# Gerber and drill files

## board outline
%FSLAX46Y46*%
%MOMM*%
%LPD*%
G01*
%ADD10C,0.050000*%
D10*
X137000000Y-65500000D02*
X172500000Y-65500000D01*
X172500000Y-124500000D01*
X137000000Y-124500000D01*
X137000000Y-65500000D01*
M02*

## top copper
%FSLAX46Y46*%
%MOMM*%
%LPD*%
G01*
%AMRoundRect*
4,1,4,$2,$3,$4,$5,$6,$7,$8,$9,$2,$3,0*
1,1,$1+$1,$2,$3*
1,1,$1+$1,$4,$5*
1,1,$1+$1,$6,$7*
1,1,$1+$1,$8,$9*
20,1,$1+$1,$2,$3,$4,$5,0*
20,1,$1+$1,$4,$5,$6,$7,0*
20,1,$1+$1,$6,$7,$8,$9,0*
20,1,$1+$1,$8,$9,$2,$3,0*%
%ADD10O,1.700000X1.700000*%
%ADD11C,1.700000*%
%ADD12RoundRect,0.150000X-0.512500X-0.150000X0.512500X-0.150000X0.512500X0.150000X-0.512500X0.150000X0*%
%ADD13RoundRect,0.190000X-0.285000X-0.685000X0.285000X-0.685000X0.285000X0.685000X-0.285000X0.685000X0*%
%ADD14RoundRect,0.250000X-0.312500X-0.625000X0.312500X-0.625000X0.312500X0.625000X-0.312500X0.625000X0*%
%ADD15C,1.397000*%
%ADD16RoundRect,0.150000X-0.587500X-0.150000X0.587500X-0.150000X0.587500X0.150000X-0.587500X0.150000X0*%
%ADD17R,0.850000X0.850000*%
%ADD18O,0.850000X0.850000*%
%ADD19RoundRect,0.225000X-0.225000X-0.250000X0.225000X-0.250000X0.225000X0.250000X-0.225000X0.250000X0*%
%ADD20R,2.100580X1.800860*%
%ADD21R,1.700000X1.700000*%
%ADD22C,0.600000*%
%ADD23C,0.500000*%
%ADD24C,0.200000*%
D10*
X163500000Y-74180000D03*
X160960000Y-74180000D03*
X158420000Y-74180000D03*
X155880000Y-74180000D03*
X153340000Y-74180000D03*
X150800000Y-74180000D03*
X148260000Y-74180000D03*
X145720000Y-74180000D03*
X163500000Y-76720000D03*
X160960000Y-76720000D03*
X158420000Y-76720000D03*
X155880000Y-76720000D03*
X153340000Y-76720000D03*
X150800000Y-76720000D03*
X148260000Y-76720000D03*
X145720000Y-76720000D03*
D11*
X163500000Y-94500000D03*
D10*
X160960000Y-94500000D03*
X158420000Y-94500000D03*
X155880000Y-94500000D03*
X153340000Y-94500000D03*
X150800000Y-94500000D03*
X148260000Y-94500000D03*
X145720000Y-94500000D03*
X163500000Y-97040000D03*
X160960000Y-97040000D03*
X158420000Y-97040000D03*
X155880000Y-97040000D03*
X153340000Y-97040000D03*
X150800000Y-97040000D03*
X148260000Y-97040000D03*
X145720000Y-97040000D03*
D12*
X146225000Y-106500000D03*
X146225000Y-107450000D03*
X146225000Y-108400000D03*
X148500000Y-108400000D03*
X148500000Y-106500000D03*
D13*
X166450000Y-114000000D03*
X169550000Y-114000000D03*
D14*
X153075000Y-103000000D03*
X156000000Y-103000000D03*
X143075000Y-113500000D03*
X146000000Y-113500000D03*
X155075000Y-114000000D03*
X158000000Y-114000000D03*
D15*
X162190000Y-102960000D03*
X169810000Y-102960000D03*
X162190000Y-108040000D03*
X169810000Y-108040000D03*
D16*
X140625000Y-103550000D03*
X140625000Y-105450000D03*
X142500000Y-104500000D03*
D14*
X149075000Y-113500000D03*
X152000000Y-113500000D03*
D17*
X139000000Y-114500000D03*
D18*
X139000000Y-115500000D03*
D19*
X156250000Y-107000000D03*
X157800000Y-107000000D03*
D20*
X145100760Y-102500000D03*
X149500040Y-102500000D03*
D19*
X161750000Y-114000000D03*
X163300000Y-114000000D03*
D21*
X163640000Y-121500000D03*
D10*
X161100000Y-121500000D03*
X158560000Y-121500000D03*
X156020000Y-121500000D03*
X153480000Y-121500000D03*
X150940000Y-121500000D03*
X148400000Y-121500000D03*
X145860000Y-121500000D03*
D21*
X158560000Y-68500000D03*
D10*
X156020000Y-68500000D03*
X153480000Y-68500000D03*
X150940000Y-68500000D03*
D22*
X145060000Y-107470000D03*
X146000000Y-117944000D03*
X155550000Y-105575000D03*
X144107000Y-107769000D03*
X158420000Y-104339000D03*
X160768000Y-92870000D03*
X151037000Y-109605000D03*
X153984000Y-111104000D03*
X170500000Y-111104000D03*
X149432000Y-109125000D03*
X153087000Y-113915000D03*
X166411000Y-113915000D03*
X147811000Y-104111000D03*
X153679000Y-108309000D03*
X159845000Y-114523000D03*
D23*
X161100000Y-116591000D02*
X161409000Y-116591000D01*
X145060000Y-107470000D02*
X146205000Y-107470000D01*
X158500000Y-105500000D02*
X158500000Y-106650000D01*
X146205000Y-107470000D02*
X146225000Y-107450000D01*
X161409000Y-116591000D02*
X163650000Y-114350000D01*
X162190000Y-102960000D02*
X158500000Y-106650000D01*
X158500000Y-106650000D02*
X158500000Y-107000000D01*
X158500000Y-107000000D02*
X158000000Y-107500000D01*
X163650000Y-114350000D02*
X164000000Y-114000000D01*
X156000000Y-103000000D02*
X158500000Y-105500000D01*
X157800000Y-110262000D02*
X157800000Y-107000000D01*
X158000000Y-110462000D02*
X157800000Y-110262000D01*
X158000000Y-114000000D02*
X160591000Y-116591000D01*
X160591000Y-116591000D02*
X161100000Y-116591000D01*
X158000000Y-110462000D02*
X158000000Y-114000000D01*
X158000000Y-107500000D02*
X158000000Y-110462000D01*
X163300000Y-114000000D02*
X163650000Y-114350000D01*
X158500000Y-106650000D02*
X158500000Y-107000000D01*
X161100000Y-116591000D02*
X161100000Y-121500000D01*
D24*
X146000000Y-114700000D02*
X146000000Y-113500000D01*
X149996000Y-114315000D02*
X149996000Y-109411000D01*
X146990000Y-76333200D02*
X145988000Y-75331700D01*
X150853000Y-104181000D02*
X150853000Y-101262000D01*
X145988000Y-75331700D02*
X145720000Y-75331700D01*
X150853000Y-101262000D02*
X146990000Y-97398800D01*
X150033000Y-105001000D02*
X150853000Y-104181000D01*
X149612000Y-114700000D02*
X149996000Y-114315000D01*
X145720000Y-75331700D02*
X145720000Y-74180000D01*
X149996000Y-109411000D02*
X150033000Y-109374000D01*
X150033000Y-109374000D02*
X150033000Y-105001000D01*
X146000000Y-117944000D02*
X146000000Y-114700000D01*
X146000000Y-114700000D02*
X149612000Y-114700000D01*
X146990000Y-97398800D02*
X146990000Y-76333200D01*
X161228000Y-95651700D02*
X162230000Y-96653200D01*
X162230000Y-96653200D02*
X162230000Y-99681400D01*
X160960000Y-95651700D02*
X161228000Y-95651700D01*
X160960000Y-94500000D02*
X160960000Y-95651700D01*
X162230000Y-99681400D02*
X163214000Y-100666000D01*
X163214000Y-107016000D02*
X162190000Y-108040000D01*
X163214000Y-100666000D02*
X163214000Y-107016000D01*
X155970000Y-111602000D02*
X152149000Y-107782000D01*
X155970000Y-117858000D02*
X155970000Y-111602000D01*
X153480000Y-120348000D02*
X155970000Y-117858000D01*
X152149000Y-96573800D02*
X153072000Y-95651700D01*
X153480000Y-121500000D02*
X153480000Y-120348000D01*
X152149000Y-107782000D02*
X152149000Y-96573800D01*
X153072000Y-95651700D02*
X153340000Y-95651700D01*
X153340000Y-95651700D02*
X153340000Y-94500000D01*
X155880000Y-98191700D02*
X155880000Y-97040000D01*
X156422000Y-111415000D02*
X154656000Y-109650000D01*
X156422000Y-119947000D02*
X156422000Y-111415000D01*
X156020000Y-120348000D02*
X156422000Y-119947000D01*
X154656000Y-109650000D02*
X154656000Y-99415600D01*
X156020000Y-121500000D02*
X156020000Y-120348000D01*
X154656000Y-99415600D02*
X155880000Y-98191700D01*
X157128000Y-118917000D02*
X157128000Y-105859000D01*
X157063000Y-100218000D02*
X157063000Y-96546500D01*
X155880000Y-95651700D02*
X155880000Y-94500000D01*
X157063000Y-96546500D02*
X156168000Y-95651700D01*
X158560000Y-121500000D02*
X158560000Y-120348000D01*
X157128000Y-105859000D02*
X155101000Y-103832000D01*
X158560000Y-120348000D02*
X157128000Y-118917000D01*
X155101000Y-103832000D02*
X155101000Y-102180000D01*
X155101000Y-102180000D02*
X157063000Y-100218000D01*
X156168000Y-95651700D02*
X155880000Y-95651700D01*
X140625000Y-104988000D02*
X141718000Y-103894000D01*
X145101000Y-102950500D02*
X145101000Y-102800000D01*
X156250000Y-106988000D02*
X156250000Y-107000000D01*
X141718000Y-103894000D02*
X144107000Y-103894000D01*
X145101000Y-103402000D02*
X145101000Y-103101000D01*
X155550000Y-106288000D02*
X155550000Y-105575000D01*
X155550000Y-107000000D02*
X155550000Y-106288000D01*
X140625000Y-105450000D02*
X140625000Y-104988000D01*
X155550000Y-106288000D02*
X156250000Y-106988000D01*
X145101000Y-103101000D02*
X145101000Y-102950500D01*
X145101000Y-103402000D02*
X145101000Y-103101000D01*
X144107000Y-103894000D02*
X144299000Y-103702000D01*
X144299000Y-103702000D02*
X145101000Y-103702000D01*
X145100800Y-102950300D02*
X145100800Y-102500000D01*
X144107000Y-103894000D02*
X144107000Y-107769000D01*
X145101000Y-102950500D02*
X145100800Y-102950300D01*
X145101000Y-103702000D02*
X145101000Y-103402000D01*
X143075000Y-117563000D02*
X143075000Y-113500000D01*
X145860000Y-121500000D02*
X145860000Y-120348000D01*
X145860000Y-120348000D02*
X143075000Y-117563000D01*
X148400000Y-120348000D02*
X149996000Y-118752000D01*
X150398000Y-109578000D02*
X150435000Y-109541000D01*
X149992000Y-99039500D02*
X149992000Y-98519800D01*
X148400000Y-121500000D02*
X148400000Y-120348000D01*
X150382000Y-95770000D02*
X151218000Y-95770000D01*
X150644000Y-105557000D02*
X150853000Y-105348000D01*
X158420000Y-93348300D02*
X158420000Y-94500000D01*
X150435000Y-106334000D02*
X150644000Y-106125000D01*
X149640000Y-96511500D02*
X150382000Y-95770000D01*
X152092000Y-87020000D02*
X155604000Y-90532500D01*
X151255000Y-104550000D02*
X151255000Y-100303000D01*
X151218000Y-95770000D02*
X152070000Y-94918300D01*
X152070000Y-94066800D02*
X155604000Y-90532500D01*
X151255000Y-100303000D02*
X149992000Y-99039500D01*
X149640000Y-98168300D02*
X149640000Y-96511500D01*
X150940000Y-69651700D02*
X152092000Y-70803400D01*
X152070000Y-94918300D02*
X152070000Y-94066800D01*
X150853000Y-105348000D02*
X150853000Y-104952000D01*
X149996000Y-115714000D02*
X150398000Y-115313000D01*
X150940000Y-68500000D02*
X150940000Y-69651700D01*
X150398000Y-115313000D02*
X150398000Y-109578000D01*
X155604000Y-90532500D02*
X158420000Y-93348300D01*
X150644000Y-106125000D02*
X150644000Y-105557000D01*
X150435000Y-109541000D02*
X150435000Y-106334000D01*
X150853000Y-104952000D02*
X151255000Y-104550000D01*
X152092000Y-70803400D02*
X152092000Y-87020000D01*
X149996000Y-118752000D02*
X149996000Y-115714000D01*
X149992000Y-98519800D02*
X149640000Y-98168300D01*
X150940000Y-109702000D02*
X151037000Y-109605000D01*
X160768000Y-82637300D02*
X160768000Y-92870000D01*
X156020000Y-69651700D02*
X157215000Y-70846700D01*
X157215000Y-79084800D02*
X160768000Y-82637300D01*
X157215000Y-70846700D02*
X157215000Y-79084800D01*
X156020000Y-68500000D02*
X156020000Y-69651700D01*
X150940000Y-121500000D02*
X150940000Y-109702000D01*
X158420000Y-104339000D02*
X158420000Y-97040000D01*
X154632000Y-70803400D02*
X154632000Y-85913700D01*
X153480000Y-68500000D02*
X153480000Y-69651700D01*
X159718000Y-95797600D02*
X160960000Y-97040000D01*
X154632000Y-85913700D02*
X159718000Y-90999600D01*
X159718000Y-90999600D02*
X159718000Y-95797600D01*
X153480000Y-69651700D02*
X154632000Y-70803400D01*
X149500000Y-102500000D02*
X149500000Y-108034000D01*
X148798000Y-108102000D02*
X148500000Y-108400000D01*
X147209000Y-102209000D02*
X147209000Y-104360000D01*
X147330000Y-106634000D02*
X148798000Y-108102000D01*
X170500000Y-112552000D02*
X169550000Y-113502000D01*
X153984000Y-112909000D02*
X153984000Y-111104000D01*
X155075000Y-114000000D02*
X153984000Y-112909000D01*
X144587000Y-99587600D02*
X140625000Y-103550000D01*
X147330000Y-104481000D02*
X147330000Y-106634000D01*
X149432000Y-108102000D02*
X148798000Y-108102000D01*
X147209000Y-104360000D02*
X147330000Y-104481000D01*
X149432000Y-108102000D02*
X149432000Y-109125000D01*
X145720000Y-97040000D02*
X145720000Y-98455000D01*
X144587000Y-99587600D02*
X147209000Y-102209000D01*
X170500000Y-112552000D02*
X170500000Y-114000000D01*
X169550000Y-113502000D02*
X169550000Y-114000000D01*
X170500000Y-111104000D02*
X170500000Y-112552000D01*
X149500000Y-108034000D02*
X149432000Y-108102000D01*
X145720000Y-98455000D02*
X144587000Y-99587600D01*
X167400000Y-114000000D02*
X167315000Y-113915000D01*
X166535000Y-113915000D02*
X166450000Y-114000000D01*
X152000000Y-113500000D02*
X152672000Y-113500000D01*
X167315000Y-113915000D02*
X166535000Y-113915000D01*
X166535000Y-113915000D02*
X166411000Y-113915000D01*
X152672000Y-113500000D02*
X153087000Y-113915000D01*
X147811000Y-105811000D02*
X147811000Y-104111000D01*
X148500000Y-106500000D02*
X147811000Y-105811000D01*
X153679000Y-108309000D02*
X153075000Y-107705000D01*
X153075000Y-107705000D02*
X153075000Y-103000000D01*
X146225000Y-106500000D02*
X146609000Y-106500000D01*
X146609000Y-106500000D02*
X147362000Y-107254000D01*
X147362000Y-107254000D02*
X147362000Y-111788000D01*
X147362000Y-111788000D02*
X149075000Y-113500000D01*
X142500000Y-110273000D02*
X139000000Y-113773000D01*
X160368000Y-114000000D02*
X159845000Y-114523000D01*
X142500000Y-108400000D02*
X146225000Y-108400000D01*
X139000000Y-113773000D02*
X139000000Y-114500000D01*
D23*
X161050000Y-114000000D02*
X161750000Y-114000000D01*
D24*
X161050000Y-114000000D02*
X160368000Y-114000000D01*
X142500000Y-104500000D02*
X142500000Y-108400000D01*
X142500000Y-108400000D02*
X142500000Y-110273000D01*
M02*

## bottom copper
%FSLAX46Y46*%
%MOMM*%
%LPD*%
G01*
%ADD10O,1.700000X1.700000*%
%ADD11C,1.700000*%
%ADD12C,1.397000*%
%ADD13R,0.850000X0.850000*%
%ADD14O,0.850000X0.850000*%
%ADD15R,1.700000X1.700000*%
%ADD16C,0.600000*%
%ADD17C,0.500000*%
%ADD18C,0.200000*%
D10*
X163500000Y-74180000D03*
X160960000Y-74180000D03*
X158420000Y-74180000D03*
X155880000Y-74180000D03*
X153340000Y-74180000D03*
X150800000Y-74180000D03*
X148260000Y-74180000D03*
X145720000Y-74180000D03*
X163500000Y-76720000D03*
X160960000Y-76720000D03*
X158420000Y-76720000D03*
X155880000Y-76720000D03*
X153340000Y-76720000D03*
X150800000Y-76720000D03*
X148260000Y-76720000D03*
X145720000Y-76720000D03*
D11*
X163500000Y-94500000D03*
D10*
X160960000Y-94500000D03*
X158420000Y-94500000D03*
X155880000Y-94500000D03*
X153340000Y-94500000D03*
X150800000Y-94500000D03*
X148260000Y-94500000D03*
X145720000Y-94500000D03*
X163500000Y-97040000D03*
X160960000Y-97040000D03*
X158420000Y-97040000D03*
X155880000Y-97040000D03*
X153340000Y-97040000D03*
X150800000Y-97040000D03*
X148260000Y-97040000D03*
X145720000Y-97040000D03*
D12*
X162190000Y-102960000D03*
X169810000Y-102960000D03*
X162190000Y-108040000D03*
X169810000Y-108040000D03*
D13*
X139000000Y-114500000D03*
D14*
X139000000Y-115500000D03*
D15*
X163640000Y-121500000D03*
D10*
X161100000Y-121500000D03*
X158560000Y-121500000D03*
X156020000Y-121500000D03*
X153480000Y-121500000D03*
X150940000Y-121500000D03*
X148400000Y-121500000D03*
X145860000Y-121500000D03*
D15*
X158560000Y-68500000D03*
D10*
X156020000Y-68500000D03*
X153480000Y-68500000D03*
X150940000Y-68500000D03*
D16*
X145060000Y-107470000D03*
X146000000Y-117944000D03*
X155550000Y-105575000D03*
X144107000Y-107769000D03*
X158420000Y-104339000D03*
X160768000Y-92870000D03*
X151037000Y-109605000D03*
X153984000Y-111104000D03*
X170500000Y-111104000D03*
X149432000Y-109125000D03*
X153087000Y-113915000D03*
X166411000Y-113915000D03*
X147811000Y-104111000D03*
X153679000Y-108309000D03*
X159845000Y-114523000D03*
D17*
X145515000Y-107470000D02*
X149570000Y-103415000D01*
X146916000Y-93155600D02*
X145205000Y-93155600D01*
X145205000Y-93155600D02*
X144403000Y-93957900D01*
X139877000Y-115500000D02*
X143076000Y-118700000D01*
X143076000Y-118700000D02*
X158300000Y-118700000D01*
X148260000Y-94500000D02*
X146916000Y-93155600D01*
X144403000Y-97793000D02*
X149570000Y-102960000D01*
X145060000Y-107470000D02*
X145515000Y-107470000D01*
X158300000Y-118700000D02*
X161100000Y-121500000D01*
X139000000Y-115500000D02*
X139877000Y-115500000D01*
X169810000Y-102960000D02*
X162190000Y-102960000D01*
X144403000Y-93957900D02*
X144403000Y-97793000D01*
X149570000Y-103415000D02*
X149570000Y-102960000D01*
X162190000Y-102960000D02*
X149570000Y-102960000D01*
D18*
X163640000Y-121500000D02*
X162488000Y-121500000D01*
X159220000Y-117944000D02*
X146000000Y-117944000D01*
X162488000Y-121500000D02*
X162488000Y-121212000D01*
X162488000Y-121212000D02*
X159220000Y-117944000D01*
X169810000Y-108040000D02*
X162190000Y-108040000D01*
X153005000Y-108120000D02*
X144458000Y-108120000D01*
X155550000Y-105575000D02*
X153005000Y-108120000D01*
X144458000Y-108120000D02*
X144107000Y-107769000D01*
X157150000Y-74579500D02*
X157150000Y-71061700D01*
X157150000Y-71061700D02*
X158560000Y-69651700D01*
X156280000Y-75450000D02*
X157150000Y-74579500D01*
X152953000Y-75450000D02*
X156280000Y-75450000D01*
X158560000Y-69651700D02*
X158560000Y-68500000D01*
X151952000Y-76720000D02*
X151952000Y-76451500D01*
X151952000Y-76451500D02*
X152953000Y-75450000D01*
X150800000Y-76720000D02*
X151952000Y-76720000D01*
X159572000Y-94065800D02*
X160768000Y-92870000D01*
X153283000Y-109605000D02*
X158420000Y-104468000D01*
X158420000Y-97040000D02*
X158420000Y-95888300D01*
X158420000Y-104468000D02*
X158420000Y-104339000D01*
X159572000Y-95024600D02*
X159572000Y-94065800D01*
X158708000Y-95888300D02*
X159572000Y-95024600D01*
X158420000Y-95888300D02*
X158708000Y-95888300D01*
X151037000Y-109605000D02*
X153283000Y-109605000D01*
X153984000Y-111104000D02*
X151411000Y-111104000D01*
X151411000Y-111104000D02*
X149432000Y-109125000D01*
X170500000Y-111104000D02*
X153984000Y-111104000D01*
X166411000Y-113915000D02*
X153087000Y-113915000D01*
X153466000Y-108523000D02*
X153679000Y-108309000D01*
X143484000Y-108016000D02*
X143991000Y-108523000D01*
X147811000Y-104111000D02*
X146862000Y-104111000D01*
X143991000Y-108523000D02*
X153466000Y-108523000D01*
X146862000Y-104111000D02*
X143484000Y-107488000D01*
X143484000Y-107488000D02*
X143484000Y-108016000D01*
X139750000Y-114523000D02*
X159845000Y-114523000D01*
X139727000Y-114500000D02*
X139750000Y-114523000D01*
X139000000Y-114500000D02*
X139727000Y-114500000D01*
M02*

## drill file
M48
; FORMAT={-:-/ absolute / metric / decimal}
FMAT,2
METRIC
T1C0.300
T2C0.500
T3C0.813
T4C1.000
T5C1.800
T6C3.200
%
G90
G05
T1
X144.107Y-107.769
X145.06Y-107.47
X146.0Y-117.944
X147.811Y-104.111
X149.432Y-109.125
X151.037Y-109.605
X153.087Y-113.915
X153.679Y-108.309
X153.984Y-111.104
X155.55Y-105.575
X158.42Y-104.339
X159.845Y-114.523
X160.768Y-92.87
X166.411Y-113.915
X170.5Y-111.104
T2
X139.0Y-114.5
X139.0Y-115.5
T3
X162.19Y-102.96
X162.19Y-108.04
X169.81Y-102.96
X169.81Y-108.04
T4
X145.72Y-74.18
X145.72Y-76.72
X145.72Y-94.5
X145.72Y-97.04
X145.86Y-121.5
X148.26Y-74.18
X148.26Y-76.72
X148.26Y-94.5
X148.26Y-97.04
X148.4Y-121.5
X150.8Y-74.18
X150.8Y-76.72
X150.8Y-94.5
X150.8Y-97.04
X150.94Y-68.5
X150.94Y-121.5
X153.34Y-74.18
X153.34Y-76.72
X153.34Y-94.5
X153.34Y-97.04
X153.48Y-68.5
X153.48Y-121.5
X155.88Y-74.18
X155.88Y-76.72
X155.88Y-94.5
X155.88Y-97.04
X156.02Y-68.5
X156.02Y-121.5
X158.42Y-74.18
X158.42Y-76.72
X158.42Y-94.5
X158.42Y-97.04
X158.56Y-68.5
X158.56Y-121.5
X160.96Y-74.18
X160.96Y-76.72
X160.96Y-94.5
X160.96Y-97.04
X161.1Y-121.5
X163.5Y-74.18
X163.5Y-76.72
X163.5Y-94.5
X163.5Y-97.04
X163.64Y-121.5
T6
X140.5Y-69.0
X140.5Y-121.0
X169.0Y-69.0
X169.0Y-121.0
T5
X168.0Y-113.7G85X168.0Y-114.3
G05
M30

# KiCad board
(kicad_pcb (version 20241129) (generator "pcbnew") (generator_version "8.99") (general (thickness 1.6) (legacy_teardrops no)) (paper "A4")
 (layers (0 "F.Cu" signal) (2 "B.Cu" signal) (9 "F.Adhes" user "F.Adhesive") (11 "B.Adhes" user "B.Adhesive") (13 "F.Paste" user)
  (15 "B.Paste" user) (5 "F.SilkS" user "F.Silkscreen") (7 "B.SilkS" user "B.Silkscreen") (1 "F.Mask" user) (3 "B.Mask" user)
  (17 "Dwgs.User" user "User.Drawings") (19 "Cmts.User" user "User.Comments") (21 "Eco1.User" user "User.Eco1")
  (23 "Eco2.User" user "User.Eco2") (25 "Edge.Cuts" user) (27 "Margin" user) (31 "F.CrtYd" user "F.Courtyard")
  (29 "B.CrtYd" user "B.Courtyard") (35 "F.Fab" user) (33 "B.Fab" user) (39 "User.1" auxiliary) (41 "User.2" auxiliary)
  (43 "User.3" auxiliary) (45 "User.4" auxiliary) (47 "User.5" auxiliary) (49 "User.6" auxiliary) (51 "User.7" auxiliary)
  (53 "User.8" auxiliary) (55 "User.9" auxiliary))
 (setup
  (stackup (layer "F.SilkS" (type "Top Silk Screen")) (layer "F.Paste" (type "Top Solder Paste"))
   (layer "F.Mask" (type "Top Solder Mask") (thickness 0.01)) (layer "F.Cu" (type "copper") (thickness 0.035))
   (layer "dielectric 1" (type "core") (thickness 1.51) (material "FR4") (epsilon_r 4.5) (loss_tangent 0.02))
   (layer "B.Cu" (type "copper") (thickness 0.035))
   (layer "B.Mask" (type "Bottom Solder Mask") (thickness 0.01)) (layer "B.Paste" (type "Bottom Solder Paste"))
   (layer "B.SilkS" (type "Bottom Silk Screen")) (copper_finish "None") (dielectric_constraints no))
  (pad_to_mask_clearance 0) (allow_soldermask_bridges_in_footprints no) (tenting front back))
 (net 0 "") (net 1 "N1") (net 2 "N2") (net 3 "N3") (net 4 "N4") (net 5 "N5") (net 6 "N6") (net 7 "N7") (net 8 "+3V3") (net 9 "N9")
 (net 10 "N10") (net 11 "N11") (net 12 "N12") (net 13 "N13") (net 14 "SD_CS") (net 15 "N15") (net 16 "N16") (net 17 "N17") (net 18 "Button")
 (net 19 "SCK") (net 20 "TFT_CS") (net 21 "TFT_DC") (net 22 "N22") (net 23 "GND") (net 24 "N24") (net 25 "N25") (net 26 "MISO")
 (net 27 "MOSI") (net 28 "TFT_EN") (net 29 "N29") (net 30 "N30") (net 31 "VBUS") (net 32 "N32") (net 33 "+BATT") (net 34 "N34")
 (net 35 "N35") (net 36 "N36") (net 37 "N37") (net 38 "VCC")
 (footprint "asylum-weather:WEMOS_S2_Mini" (layer "F.Cu") (at 156 85.61 -90)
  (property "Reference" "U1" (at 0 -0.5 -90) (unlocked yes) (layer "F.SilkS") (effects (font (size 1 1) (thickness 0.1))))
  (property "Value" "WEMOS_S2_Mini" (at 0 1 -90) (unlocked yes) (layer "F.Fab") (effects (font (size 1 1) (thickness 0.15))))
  (pad "1" thru_hole oval (at -11.43 -7.5 270) (size 1.7 1.7) (drill 1) (layers "*.Cu" "*.Mask") (remove_unused_layers no) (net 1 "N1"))
  (pad "2" thru_hole oval (at -11.43 -4.96 270) (size 1.7 1.7) (drill 1) (layers "*.Cu" "*.Mask") (remove_unused_layers no) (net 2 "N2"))
  (pad "3" thru_hole oval (at -11.43 -2.42 270) (size 1.7 1.7) (drill 1) (layers "*.Cu" "*.Mask") (remove_unused_layers no) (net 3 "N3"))
  (pad "4" thru_hole oval (at -11.43 0.12 270) (size 1.7 1.7) (drill 1) (layers "*.Cu" "*.Mask") (remove_unused_layers no) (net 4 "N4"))
  (pad "5" thru_hole oval (at -11.43 2.66 270) (size 1.7 1.7) (drill 1) (layers "*.Cu" "*.Mask") (remove_unused_layers no) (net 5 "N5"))
  (pad "6" thru_hole oval (at -11.43 5.2 270) (size 1.7 1.7) (drill 1) (layers "*.Cu" "*.Mask") (remove_unused_layers no) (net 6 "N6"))
  (pad "7" thru_hole oval (at -11.43 7.74 270) (size 1.7 1.7) (drill 1) (layers "*.Cu" "*.Mask") (remove_unused_layers no) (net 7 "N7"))
  (pad "8" thru_hole oval (at -11.43 10.28 270) (size 1.7 1.7) (drill 1) (layers "*.Cu" "*.Mask") (remove_unused_layers no) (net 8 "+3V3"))
  (pad "9" thru_hole oval (at -8.89 -7.5 270) (size 1.7 1.7) (drill 1) (layers "*.Cu" "*.Mask") (remove_unused_layers no) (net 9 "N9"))
  (pad "10" thru_hole oval (at -8.89 -4.96 270) (size 1.7 1.7) (drill 1) (layers "*.Cu" "*.Mask") (remove_unused_layers no) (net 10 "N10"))
  (pad "11" thru_hole oval (at -8.89 -2.42 270) (size 1.7 1.7) (drill 1) (layers "*.Cu" "*.Mask") (remove_unused_layers no) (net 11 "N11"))
  (pad "12" thru_hole oval (at -8.89 0.12 270) (size 1.7 1.7) (drill 1) (layers "*.Cu" "*.Mask") (remove_unused_layers no) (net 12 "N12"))
  (pad "13" thru_hole oval (at -8.89 2.66 270) (size 1.7 1.7) (drill 1) (layers "*.Cu" "*.Mask") (remove_unused_layers no) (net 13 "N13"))
  (pad "14" thru_hole oval (at -8.89 5.2 270) (size 1.7 1.7) (drill 1) (layers "*.Cu" "*.Mask") (remove_unused_layers no) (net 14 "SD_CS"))
  (pad "15" thru_hole oval (at -8.89 7.74 270) (size 1.7 1.7) (drill 1) (layers "*.Cu" "*.Mask") (remove_unused_layers no) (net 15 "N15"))
  (pad "16" thru_hole oval (at -8.89 10.28 270) (size 1.7 1.7) (drill 1) (layers "*.Cu" "*.Mask") (remove_unused_layers no) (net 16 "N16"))
  (pad "17" thru_hole circle (at 8.89 -7.5 270) (size 1.7 1.7) (drill 1) (layers "*.Cu" "*.Mask") (remove_unused_layers no) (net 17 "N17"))
  (pad "18" thru_hole oval (at 8.89 -4.96 270) (size 1.7 1.7) (drill 1) (layers "*.Cu" "*.Mask") (remove_unused_layers no) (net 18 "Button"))
  (pad "19" thru_hole oval (at 8.89 -2.42 270) (size 1.7 1.7) (drill 1) (layers "*.Cu" "*.Mask") (remove_unused_layers no) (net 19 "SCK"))
  (pad "20" thru_hole oval (at 8.89 0.12 270) (size 1.7 1.7) (drill 1) (layers "*.Cu" "*.Mask") (remove_unused_layers no) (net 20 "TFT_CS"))
  (pad "21" thru_hole oval (at 8.89 2.66 270) (size 1.7 1.7) (drill 1) (layers "*.Cu" "*.Mask") (remove_unused_layers no) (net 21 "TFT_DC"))
  (pad "22" thru_hole oval (at 8.89 5.2 270) (size 1.7 1.7) (drill 1) (layers "*.Cu" "*.Mask") (remove_unused_layers no) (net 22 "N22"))
  (pad "23" thru_hole oval (at 8.89 7.74 270) (size 1.7 1.7) (drill 1) (layers "*.Cu" "*.Mask") (remove_unused_layers no) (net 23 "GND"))
  (pad "24" thru_hole oval (at 8.89 10.28 270) (size 1.7 1.7) (drill 1) (layers "*.Cu" "*.Mask") (remove_unused_layers no) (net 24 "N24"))
  (pad "25" thru_hole oval (at 11.43 -7.5 270) (size 1.7 1.7) (drill 1) (layers "*.Cu" "*.Mask") (remove_unused_layers no) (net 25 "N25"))
  (pad "26" thru_hole oval (at 11.43 -4.96 270) (size 1.7 1.7) (drill 1) (layers "*.Cu" "*.Mask") (remove_unused_layers no) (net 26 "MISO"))
  (pad "27" thru_hole oval (at 11.43 -2.42 270) (size 1.7 1.7) (drill 1) (layers "*.Cu" "*.Mask") (remove_unused_layers no) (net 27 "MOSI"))
  (pad "28" thru_hole oval (at 11.43 0.12 270) (size 1.7 1.7) (drill 1) (layers "*.Cu" "*.Mask") (remove_unused_layers no) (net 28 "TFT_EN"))
  (pad "29" thru_hole oval (at 11.43 2.66 270) (size 1.7 1.7) (drill 1) (layers "*.Cu" "*.Mask") (remove_unused_layers no) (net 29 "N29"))
  (pad "30" thru_hole oval (at 11.43 5.2 270) (size 1.7 1.7) (drill 1) (layers "*.Cu" "*.Mask") (remove_unused_layers no) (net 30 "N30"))
  (pad "31" thru_hole oval (at 11.43 7.74 270) (size 1.7 1.7) (drill 1) (layers "*.Cu" "*.Mask") (remove_unused_layers no))
  (pad "32" thru_hole oval (at 11.43 10.28 270) (size 1.7 1.7) (drill 1) (layers "*.Cu" "*.Mask") (remove_unused_layers no) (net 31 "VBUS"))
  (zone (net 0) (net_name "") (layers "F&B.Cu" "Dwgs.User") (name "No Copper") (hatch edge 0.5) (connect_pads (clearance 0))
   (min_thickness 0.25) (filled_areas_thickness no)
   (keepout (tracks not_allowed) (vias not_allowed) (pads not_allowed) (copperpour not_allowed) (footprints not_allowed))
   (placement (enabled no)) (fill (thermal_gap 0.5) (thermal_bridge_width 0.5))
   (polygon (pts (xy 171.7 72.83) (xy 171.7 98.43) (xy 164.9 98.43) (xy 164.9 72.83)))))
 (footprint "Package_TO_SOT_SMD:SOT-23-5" (layer "F.Cu") (at 147.3625 107.45)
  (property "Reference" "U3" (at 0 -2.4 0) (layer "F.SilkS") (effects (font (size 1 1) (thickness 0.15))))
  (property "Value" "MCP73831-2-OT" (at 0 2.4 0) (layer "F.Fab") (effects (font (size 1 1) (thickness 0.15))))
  (pad "1" smd roundrect (at -1.1375 -0.95) (size 1.325 0.6) (layers "F.Cu" "F.Mask" "F.Paste") (roundrect_rratio 0.25) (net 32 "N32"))
  (pad "2" smd roundrect (at -1.1375 0) (size 1.325 0.6) (layers "F.Cu" "F.Mask" "F.Paste") (roundrect_rratio 0.25) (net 23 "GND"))
  (pad "3" smd roundrect (at -1.1375 0.95) (size 1.325 0.6) (layers "F.Cu" "F.Mask" "F.Paste") (roundrect_rratio 0.25) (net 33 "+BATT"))
  (pad "4" smd roundrect (at 1.1375 0.95) (size 1.325 0.6) (layers "F.Cu" "F.Mask" "F.Paste") (roundrect_rratio 0.25) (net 31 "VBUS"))
  (pad "5" smd roundrect (at 1.1375 -0.95) (size 1.325 0.6) (layers "F.Cu" "F.Mask" "F.Paste") (roundrect_rratio 0.25) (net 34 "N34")))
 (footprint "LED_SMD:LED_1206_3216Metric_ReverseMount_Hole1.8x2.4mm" (layer "F.Cu") (at 168 114)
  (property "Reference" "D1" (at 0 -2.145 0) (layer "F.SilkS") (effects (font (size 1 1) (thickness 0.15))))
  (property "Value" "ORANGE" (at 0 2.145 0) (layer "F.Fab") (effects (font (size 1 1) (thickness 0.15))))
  (pad "" np_thru_hole oval (at 0 0) (size 1.8 2.4) (drill oval 1.8 2.4) (layers "*.Cu" "*.Mask"))
  (pad "1" smd roundrect (at -1.55 0) (size 0.95 1.75) (layers "F.Cu" "F.Mask" "F.Paste") (roundrect_rratio 0.2) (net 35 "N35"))
  (pad "2" smd roundrect (at 1.55 0) (size 0.95 1.75) (layers "F.Cu" "F.Mask" "F.Paste") (roundrect_rratio 0.2) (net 31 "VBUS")))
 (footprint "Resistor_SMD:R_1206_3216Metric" (layer "F.Cu") (at 154.5375 103)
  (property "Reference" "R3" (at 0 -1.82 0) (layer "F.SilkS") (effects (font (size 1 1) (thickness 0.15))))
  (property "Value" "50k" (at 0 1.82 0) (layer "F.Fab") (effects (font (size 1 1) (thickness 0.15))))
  (pad "1" smd roundrect (at -1.4625 0) (size 1.125 1.75) (layers "F.Cu" "F.Mask" "F.Paste") (roundrect_rratio 0.222222) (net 34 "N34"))
  (pad "2" smd roundrect (at 1.4625 0) (size 1.125 1.75) (layers "F.Cu" "F.Mask" "F.Paste") (roundrect_rratio 0.222222) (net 23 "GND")))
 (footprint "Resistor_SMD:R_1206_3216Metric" (layer "F.Cu") (at 144.5375 113.5)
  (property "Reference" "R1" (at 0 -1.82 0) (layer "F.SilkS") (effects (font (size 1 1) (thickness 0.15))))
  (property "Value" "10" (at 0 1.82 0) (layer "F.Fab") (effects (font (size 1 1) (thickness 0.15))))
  (pad "1" smd roundrect (at -1.4625 0) (size 1.125 1.75) (layers "F.Cu" "F.Mask" "F.Paste") (roundrect_rratio 0.222222) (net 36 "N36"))
  (pad "2" smd roundrect (at 1.4625 0) (size 1.125 1.75) (layers "F.Cu" "F.Mask" "F.Paste") (roundrect_rratio 0.222222) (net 8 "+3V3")))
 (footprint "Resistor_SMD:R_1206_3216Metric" (layer "F.Cu") (at 156.5375 114)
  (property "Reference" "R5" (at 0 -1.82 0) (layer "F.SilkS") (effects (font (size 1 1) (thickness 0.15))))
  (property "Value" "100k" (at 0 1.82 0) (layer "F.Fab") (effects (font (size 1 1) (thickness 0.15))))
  (pad "1" smd roundrect (at -1.4625 0) (size 1.125 1.75) (layers "F.Cu" "F.Mask" "F.Paste") (roundrect_rratio 0.222222) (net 31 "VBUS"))
  (pad "2" smd roundrect (at 1.4625 0) (size 1.125 1.75) (layers "F.Cu" "F.Mask" "F.Paste") (roundrect_rratio 0.222222) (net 23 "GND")))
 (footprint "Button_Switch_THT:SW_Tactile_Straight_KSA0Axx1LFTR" (layer "F.Cu") (at 162.19 102.96)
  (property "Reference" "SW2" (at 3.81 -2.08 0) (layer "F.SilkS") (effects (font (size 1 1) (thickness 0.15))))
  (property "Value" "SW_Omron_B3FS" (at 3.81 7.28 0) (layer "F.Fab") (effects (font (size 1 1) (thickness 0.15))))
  (pad "1" thru_hole circle (at 0 0) (size 1.397 1.397) (drill 0.8128) (layers "*.Cu" "*.Mask") (remove_unused_layers no) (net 23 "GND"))
  (pad "1" thru_hole circle (at 7.62 0) (size 1.397 1.397) (drill 0.8128) (layers "*.Cu" "*.Mask") (remove_unused_layers no) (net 23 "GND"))
  (pad "2" thru_hole circle (at 0 5.08) (size 1.397 1.397) (drill 0.8128) (layers "*.Cu" "*.Mask") (remove_unused_layers no)
   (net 18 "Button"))
  (pad "2" thru_hole circle (at 7.62 5.08) (size 1.397 1.397) (drill 0.8128) (layers "*.Cu" "*.Mask") (remove_unused_layers no)
   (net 18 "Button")))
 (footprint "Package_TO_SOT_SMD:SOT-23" (layer "F.Cu") (at 141.5625 104.5)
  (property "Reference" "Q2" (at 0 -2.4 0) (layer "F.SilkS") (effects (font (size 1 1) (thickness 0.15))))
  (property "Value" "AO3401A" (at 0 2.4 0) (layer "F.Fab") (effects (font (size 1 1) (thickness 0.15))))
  (pad "1" smd roundrect (at -0.9375 -0.95) (size 1.475 0.6) (layers "F.Cu" "F.Mask" "F.Paste") (roundrect_rratio 0.25) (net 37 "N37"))
  (pad "2" smd roundrect (at -0.9375 0.95) (size 1.475 0.6) (layers "F.Cu" "F.Mask" "F.Paste") (roundrect_rratio 0.25) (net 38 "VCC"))
  (pad "3" smd roundrect (at 0.9375 0) (size 1.475 0.6) (layers "F.Cu" "F.Mask" "F.Paste") (roundrect_rratio 0.25) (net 33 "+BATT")))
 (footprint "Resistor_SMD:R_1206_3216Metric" (layer "F.Cu") (at 150.5375 113.5)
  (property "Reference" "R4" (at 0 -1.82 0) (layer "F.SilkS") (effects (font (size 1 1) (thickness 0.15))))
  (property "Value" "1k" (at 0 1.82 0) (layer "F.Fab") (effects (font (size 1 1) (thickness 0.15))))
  (pad "1" smd roundrect (at -1.4625 0) (size 1.125 1.75) (layers "F.Cu" "F.Mask" "F.Paste") (roundrect_rratio 0.222222) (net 32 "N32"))
  (pad "2" smd roundrect (at 1.4625 0) (size 1.125 1.75) (layers "F.Cu" "F.Mask" "F.Paste") (roundrect_rratio 0.222222) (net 35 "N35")))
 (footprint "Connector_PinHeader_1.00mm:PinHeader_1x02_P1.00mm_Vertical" (layer "F.Cu") (at 139 114.5)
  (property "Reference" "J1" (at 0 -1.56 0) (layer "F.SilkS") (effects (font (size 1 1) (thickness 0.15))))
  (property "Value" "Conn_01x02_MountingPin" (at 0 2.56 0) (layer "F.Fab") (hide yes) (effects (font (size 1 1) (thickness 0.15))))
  (pad "1" thru_hole rect (at 0 0) (size 0.85 0.85) (drill 0.5) (layers "*.Cu" "*.Mask") (remove_unused_layers no) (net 33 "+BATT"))
  (pad "2" thru_hole oval (at 0 1) (size 0.85 0.85) (drill 0.5) (layers "*.Cu" "*.Mask") (remove_unused_layers no) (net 23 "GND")))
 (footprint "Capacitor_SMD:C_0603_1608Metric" (layer "F.Cu") (at 157.025 107)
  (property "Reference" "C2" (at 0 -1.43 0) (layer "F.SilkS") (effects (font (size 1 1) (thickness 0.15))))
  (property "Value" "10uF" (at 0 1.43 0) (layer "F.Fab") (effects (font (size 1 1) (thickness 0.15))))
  (pad "1" smd roundrect (at -0.775 0) (size 0.9 0.95) (layers "F.Cu" "F.Mask" "F.Paste") (roundrect_rratio 0.25) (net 38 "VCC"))
  (pad "2" smd roundrect (at 0.775 0) (size 0.9 0.95) (layers "F.Cu" "F.Mask" "F.Paste") (roundrect_rratio 0.25) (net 23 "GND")))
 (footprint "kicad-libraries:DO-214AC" (layer "F.Cu") (at 147.3004 102.5)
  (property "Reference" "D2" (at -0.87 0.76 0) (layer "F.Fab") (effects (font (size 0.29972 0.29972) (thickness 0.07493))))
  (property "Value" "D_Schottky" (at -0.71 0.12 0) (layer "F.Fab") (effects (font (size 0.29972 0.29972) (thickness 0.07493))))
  (pad "1" smd rect (at -2.19964 0) (size 2.10058 1.80086) (layers "F.Cu" "F.Mask" "F.Paste") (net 38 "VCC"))
  (pad "2" smd rect (at 2.19964 0) (size 2.10058 1.80086) (layers "F.Cu" "F.Mask" "F.Paste") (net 31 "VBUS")))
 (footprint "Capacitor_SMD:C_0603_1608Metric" (layer "F.Cu") (at 162.525 114)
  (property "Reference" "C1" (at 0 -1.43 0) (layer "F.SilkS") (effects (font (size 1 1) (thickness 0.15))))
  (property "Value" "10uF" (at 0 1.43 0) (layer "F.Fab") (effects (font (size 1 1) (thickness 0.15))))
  (pad "1" smd roundrect (at -0.775 0) (size 0.9 0.95) (layers "F.Cu" "F.Mask" "F.Paste") (roundrect_rratio 0.25) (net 33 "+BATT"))
  (pad "2" smd roundrect (at 0.775 0) (size 0.9 0.95) (layers "F.Cu" "F.Mask" "F.Paste") (roundrect_rratio 0.25) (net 23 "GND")))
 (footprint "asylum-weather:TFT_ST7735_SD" (layer "B.Cu") (at 155 101.5 90)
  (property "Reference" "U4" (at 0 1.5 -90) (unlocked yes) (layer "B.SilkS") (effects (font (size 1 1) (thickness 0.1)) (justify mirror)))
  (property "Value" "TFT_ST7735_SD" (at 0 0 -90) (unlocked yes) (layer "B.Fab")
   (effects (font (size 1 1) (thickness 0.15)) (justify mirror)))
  (pad "" np_thru_hole circle (at -19.5 -14.5 90) (size 3.2 3.2) (drill 3.2) (layers "F&B.Cu" "*.Mask"))
  (pad "" np_thru_hole circle (at -19.5 14 90) (size 3.2 3.2) (drill 3.2) (layers "F&B.Cu" "*.Mask"))
  (pad "" np_thru_hole circle (at 32.5 -14.5 90) (size 3.2 3.2) (drill 3.2) (layers "F&B.Cu" "*.Mask"))
  (pad "" np_thru_hole circle (at 32.5 14 90) (size 3.2 3.2) (drill 3.2) (layers "F&B.Cu" "*.Mask"))
  (pad "1" thru_hole rect (at -20 8.64 90) (size 1.7 1.7) (drill 1) (layers "F&B.Cu" "*.Mask") (remove_unused_layers no) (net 8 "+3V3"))
  (pad "2" thru_hole oval (at -20 6.1 90) (size 1.7 1.7) (drill 1) (layers "F&B.Cu" "*.Mask") (remove_unused_layers no) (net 23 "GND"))
  (pad "3" thru_hole oval (at -20 3.56 90) (size 1.7 1.7) (drill 1) (layers "F&B.Cu" "*.Mask") (remove_unused_layers no) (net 20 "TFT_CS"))
  (pad "4" thru_hole oval (at -20 1.02 90) (size 1.7 1.7) (drill 1) (layers "F&B.Cu" "*.Mask") (remove_unused_layers no) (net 28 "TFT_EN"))
  (pad "5" thru_hole oval (at -20 -1.52 90) (size 1.7 1.7) (drill 1) (layers "F&B.Cu" "*.Mask") (remove_unused_layers no) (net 21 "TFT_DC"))
  (pad "6" thru_hole oval (at -20 -4.06 90) (size 1.7 1.7) (drill 1) (layers "F&B.Cu" "*.Mask") (remove_unused_layers no) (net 27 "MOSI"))
  (pad "7" thru_hole oval (at -20 -6.6 90) (size 1.7 1.7) (drill 1) (layers "F&B.Cu" "*.Mask") (remove_unused_layers no) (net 19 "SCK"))
  (pad "8" thru_hole oval (at -20 -9.14 90) (size 1.7 1.7) (drill 1) (layers "F&B.Cu" "*.Mask") (remove_unused_layers no) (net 36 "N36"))
  (pad "9" thru_hole rect (at 33 3.56 90) (size 1.7 1.7) (drill 1) (layers "F&B.Cu" "*.Mask") (remove_unused_layers no) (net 14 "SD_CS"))
  (pad "10" thru_hole oval (at 33 1.02 90) (size 1.7 1.7) (drill 1) (layers "F&B.Cu" "*.Mask") (remove_unused_layers no) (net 27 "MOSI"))
  (pad "11" thru_hole oval (at 33 -1.52 90) (size 1.7 1.7) (drill 1) (layers "F&B.Cu" "*.Mask") (remove_unused_layers no) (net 26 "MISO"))
  (pad "12" thru_hole oval (at 33 -4.06 90) (size 1.7 1.7) (drill 1) (layers "F&B.Cu" "*.Mask") (remove_unused_layers no) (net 19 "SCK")))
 (gr_rect (start 137 65.5) (end 172.5 124.5) (stroke (width 0.05) (type default)) (fill no) (layer "Edge.Cuts"))
 (segment (start 161.1 116.591) (end 161.409 116.591) (width 0.5) (layer "F.Cu") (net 23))
 (segment (start 145.06 107.47) (end 146.205 107.47) (width 0.5) (layer "F.Cu") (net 23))
 (segment (start 158.5 105.5) (end 158.5 106.65) (width 0.5) (layer "F.Cu") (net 23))
 (segment (start 146.205 107.47) (end 146.225 107.45) (width 0.5) (layer "F.Cu") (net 23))
 (segment (start 161.409 116.591) (end 163.65 114.35) (width 0.5) (layer "F.Cu") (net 23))
 (segment (start 162.19 102.96) (end 158.5 106.65) (width 0.5) (layer "F.Cu") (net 23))
 (segment (start 158.5 106.65) (end 158.5 107) (width 0.5) (layer "F.Cu") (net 23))
 (segment (start 158.5 107) (end 158 107.5) (width 0.5) (layer "F.Cu") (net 23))
 (segment (start 163.65 114.35) (end 164 114) (width 0.5) (layer "F.Cu") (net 23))
 (segment (start 156 103) (end 158.5 105.5) (width 0.5) (layer "F.Cu") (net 23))
 (segment (start 157.8 110.262) (end 157.8 107) (width 0.5) (layer "F.Cu") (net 23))
 (segment (start 158 110.462) (end 157.8 110.262) (width 0.5) (layer "F.Cu") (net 23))
 (segment (start 158 114) (end 160.591 116.591) (width 0.5) (layer "F.Cu") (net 23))
 (segment (start 160.591 116.591) (end 161.1 116.591) (width 0.5) (layer "F.Cu") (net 23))
 (segment (start 158 110.462) (end 158 114) (width 0.5) (layer "F.Cu") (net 23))
 (segment (start 158 107.5) (end 158 110.462) (width 0.5) (layer "F.Cu") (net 23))
 (segment (start 163.3 114) (end 163.65 114.35) (width 0.5) (layer "F.Cu") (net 23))
 (segment (start 158.5 106.65) (end 158.5 107) (width 0.5) (layer "F.Cu") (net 23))
 (segment (start 161.1 116.591) (end 161.1 121.5) (width 0.5) (layer "F.Cu") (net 23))
 (via (at 145.06 107.47) (size 0.6) (drill 0.3) (layers "F.Cu" "B.Cu") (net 23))
 (segment (start 145.515 107.47) (end 149.57 103.415) (width 0.5) (layer "B.Cu") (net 23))
 (segment (start 146.916 93.1556) (end 145.205 93.1556) (width 0.5) (layer "B.Cu") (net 23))
 (segment (start 145.205 93.1556) (end 144.403 93.9579) (width 0.5) (layer "B.Cu") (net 23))
 (segment (start 139.877 115.5) (end 143.076 118.7) (width 0.5) (layer "B.Cu") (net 23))
 (segment (start 143.076 118.7) (end 158.3 118.7) (width 0.5) (layer "B.Cu") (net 23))
 (segment (start 148.26 94.5) (end 146.916 93.1556) (width 0.5) (layer "B.Cu") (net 23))
 (segment (start 144.403 97.793) (end 149.57 102.96) (width 0.5) (layer "B.Cu") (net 23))
 (segment (start 145.06 107.47) (end 145.515 107.47) (width 0.5) (layer "B.Cu") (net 23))
 (segment (start 158.3 118.7) (end 161.1 121.5) (width 0.5) (layer "B.Cu") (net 23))
 (segment (start 139 115.5) (end 139.877 115.5) (width 0.5) (layer "B.Cu") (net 23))
 (segment (start 169.81 102.96) (end 162.19 102.96) (width 0.5) (layer "B.Cu") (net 23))
 (segment (start 144.403 93.9579) (end 144.403 97.793) (width 0.5) (layer "B.Cu") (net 23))
 (segment (start 149.57 103.415) (end 149.57 102.96) (width 0.5) (layer "B.Cu") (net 23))
 (segment (start 162.19 102.96) (end 149.57 102.96) (width 0.5) (layer "B.Cu") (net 23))
 (segment (start 146 114.7) (end 146 113.5) (width 0.2) (layer "F.Cu") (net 8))
 (segment (start 149.996 114.315) (end 149.996 109.411) (width 0.2) (layer "F.Cu") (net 8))
 (segment (start 146.99 76.3332) (end 145.988 75.3317) (width 0.2) (layer "F.Cu") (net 8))
 (segment (start 150.853 104.181) (end 150.853 101.262) (width 0.2) (layer "F.Cu") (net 8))
 (segment (start 145.988 75.3317) (end 145.72 75.3317) (width 0.2) (layer "F.Cu") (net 8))
 (segment (start 150.853 101.262) (end 146.99 97.3988) (width 0.2) (layer "F.Cu") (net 8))
 (segment (start 150.033 105.001) (end 150.853 104.181) (width 0.2) (layer "F.Cu") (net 8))
 (segment (start 149.612 114.7) (end 149.996 114.315) (width 0.2) (layer "F.Cu") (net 8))
 (segment (start 145.72 75.3317) (end 145.72 74.18) (width 0.2) (layer "F.Cu") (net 8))
 (segment (start 149.996 109.411) (end 150.033 109.374) (width 0.2) (layer "F.Cu") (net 8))
 (segment (start 150.033 109.374) (end 150.033 105.001) (width 0.2) (layer "F.Cu") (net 8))
 (segment (start 146 117.944) (end 146 114.7) (width 0.2) (layer "F.Cu") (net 8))
 (segment (start 146 114.7) (end 149.612 114.7) (width 0.2) (layer "F.Cu") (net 8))
 (segment (start 146.99 97.3988) (end 146.99 76.3332) (width 0.2) (layer "F.Cu") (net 8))
 (via (at 146 117.944) (size 0.6) (drill 0.3) (layers "F.Cu" "B.Cu") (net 8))
 (segment (start 163.64 121.5) (end 162.488 121.5) (width 0.2) (layer "B.Cu") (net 8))
 (segment (start 159.22 117.944) (end 146 117.944) (width 0.2) (layer "B.Cu") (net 8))
 (segment (start 162.488 121.5) (end 162.488 121.212) (width 0.2) (layer "B.Cu") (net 8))
 (segment (start 162.488 121.212) (end 159.22 117.944) (width 0.2) (layer "B.Cu") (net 8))
 (segment (start 161.228 95.6517) (end 162.23 96.6532) (width 0.2) (layer "F.Cu") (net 18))
 (segment (start 162.23 96.6532) (end 162.23 99.6814) (width 0.2) (layer "F.Cu") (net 18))
 (segment (start 160.96 95.6517) (end 161.228 95.6517) (width 0.2) (layer "F.Cu") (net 18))
 (segment (start 160.96 94.5) (end 160.96 95.6517) (width 0.2) (layer "F.Cu") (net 18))
 (segment (start 162.23 99.6814) (end 163.214 100.666) (width 0.2) (layer "F.Cu") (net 18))
 (segment (start 163.214 107.016) (end 162.19 108.04) (width 0.2) (layer "F.Cu") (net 18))
 (segment (start 163.214 100.666) (end 163.214 107.016) (width 0.2) (layer "F.Cu") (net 18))
 (segment (start 169.81 108.04) (end 162.19 108.04) (width 0.2) (layer "B.Cu") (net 18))
 (segment (start 155.97 111.602) (end 152.149 107.782) (width 0.2) (layer "F.Cu") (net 21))
 (segment (start 155.97 117.858) (end 155.97 111.602) (width 0.2) (layer "F.Cu") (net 21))
 (segment (start 153.48 120.348) (end 155.97 117.858) (width 0.2) (layer "F.Cu") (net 21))
 (segment (start 152.149 96.5738) (end 153.072 95.6517) (width 0.2) (layer "F.Cu") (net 21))
 (segment (start 153.48 121.5) (end 153.48 120.348) (width 0.2) (layer "F.Cu") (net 21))
 (segment (start 152.149 107.782) (end 152.149 96.5738) (width 0.2) (layer "F.Cu") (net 21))
 (segment (start 153.072 95.6517) (end 153.34 95.6517) (width 0.2) (layer "F.Cu") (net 21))
 (segment (start 153.34 95.6517) (end 153.34 94.5) (width 0.2) (layer "F.Cu") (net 21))
 (segment (start 155.88 98.1917) (end 155.88 97.04) (width 0.2) (layer "F.Cu") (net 28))
 (segment (start 156.422 111.415) (end 154.656 109.65) (width 0.2) (layer "F.Cu") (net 28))
 (segment (start 156.422 119.947) (end 156.422 111.415) (width 0.2) (layer "F.Cu") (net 28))
 (segment (start 156.02 120.348) (end 156.422 119.947) (width 0.2) (layer "F.Cu") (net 28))
 (segment (start 154.656 109.65) (end 154.656 99.4156) (width 0.2) (layer "F.Cu") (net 28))
 (segment (start 156.02 121.5) (end 156.02 120.348) (width 0.2) (layer "F.Cu") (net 28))
 (segment (start 154.656 99.4156) (end 155.88 98.1917) (width 0.2) (layer "F.Cu") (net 28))
 (segment (start 157.128 118.917) (end 157.128 105.859) (width 0.2) (layer "F.Cu") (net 20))
 (segment (start 157.063 100.218) (end 157.063 96.5465) (width 0.2) (layer "F.Cu") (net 20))
 (segment (start 155.88 95.6517) (end 155.88 94.5) (width 0.2) (layer "F.Cu") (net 20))
 (segment (start 157.063 96.5465) (end 156.168 95.6517) (width 0.2) (layer "F.Cu") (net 20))
 (segment (start 158.56 121.5) (end 158.56 120.348) (width 0.2) (layer "F.Cu") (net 20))
 (segment (start 157.128 105.859) (end 155.101 103.832) (width 0.2) (layer "F.Cu") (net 20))
 (segment (start 158.56 120.348) (end 157.128 118.917) (width 0.2) (layer "F.Cu") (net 20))
 (segment (start 155.101 103.832) (end 155.101 102.18) (width 0.2) (layer "F.Cu") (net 20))
 (segment (start 155.101 102.18) (end 157.063 100.218) (width 0.2) (layer "F.Cu") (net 20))
 (segment (start 156.168 95.6517) (end 155.88 95.6517) (width 0.2) (layer "F.Cu") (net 20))
 (segment (start 140.625 104.988) (end 141.718 103.894) (width 0.2) (layer "F.Cu") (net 38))
 (segment (start 145.101 102.9505) (end 145.101 102.8) (width 0.2) (layer "F.Cu") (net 38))
 (segment (start 156.25 106.988) (end 156.25 107) (width 0.2) (layer "F.Cu") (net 38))
 (segment (start 141.718 103.894) (end 144.107 103.894) (width 0.2) (layer "F.Cu") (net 38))
 (segment (start 145.101 103.402) (end 145.101 103.101) (width 0.2) (layer "F.Cu") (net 38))
 (segment (start 155.55 106.288) (end 155.55 105.575) (width 0.2) (layer "F.Cu") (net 38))
 (segment (start 155.55 107) (end 155.55 106.288) (width 0.2) (layer "F.Cu") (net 38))
 (segment (start 140.625 105.45) (end 140.625 104.988) (width 0.2) (layer "F.Cu") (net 38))
 (segment (start 155.55 106.288) (end 156.25 106.988) (width 0.2) (layer "F.Cu") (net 38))
 (segment (start 145.101 103.101) (end 145.101 102.9505) (width 0.2) (layer "F.Cu") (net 38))
 (segment (start 145.101 103.402) (end 145.101 103.101) (width 0.2) (layer "F.Cu") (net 38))
 (segment (start 144.107 103.894) (end 144.299 103.702) (width 0.2) (layer "F.Cu") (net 38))
 (segment (start 144.299 103.702) (end 145.101 103.702) (width 0.2) (layer "F.Cu") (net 38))
 (segment (start 145.1008 102.9503) (end 145.1008 102.5) (width 0.2) (layer "F.Cu") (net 38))
 (segment (start 144.107 103.894) (end 144.107 107.769) (width 0.2) (layer "F.Cu") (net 38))
 (segment (start 145.101 102.9505) (end 145.1008 102.9503) (width 0.2) (layer "F.Cu") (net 38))
 (segment (start 145.101 103.702) (end 145.101 103.402) (width 0.2) (layer "F.Cu") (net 38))
 (via (at 155.55 105.575) (size 0.6) (drill 0.3) (layers "F.Cu" "B.Cu") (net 38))
 (via (at 144.107 107.769) (size 0.6) (drill 0.3) (layers "F.Cu" "B.Cu") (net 38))
 (segment (start 153.005 108.12) (end 144.458 108.12) (width 0.2) (layer "B.Cu") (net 38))
 (segment (start 155.55 105.575) (end 153.005 108.12) (width 0.2) (layer "B.Cu") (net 38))
 (segment (start 144.458 108.12) (end 144.107 107.769) (width 0.2) (layer "B.Cu") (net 38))
 (segment (start 143.075 117.563) (end 143.075 113.5) (width 0.2) (layer "F.Cu") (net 36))
 (segment (start 145.86 121.5) (end 145.86 120.348) (width 0.2) (layer "F.Cu") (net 36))
 (segment (start 145.86 120.348) (end 143.075 117.563) (width 0.2) (layer "F.Cu") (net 36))
 (segment (start 157.15 74.5795) (end 157.15 71.0617) (width 0.2) (layer "B.Cu") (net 14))
 (segment (start 157.15 71.0617) (end 158.56 69.6517) (width 0.2) (layer "B.Cu") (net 14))
 (segment (start 156.28 75.45) (end 157.15 74.5795) (width 0.2) (layer "B.Cu") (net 14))
 (segment (start 152.953 75.45) (end 156.28 75.45) (width 0.2) (layer "B.Cu") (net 14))
 (segment (start 158.56 69.6517) (end 158.56 68.5) (width 0.2) (layer "B.Cu") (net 14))
 (segment (start 151.952 76.72) (end 151.952 76.4515) (width 0.2) (layer "B.Cu") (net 14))
 (segment (start 151.952 76.4515) (end 152.953 75.45) (width 0.2) (layer "B.Cu") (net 14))
 (segment (start 150.8 76.72) (end 151.952 76.72) (width 0.2) (layer "B.Cu") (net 14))
 (segment (start 148.4 120.348) (end 149.996 118.752) (width 0.2) (layer "F.Cu") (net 19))
 (segment (start 150.398 109.578) (end 150.435 109.541) (width 0.2) (layer "F.Cu") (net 19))
 (segment (start 149.992 99.0395) (end 149.992 98.5198) (width 0.2) (layer "F.Cu") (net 19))
 (segment (start 148.4 121.5) (end 148.4 120.348) (width 0.2) (layer "F.Cu") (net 19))
 (segment (start 150.382 95.77) (end 151.218 95.77) (width 0.2) (layer "F.Cu") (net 19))
 (segment (start 150.644 105.557) (end 150.853 105.348) (width 0.2) (layer "F.Cu") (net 19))
 (segment (start 158.42 93.3483) (end 158.42 94.5) (width 0.2) (layer "F.Cu") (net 19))
 (segment (start 150.435 106.334) (end 150.644 106.125) (width 0.2) (layer "F.Cu") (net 19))
 (segment (start 149.64 96.5115) (end 150.382 95.77) (width 0.2) (layer "F.Cu") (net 19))
 (segment (start 152.092 87.02) (end 155.604 90.5325) (width 0.2) (layer "F.Cu") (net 19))
 (segment (start 151.255 104.55) (end 151.255 100.303) (width 0.2) (layer "F.Cu") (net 19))
 (segment (start 151.218 95.77) (end 152.07 94.9183) (width 0.2) (layer "F.Cu") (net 19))
 (segment (start 152.07 94.0668) (end 155.604 90.5325) (width 0.2) (layer "F.Cu") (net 19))
 (segment (start 151.255 100.303) (end 149.992 99.0395) (width 0.2) (layer "F.Cu") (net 19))
 (segment (start 149.64 98.1683) (end 149.64 96.5115) (width 0.2) (layer "F.Cu") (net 19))
 (segment (start 150.94 69.6517) (end 152.092 70.8034) (width 0.2) (layer "F.Cu") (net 19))
 (segment (start 152.07 94.9183) (end 152.07 94.0668) (width 0.2) (layer "F.Cu") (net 19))
 (segment (start 150.853 105.348) (end 150.853 104.952) (width 0.2) (layer "F.Cu") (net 19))
 (segment (start 149.996 115.714) (end 150.398 115.313) (width 0.2) (layer "F.Cu") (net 19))
 (segment (start 150.94 68.5) (end 150.94 69.6517) (width 0.2) (layer "F.Cu") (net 19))
 (segment (start 150.398 115.313) (end 150.398 109.578) (width 0.2) (layer "F.Cu") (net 19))
 (segment (start 155.604 90.5325) (end 158.42 93.3483) (width 0.2) (layer "F.Cu") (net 19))
 (segment (start 150.644 106.125) (end 150.644 105.557) (width 0.2) (layer "F.Cu") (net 19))
 (segment (start 150.435 109.541) (end 150.435 106.334) (width 0.2) (layer "F.Cu") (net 19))
 (segment (start 150.853 104.952) (end 151.255 104.55) (width 0.2) (layer "F.Cu") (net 19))
 (segment (start 152.092 70.8034) (end 152.092 87.02) (width 0.2) (layer "F.Cu") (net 19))
 (segment (start 149.996 118.752) (end 149.996 115.714) (width 0.2) (layer "F.Cu") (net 19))
 (segment (start 149.992 98.5198) (end 149.64 98.1683) (width 0.2) (layer "F.Cu") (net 19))
 (segment (start 150.94 109.702) (end 151.037 109.605) (width 0.2) (layer "F.Cu") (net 27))
 (segment (start 160.768 82.6373) (end 160.768 92.87) (width 0.2) (layer "F.Cu") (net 27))
 (segment (start 156.02 69.6517) (end 157.215 70.8467) (width 0.2) (layer "F.Cu") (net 27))
 (segment (start 157.215 79.0848) (end 160.768 82.6373) (width 0.2) (layer "F.Cu") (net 27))
 (segment (start 157.215 70.8467) (end 157.215 79.0848) (width 0.2) (layer "F.Cu") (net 27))
 (segment (start 156.02 68.5) (end 156.02 69.6517) (width 0.2) (layer "F.Cu") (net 27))
 (segment (start 150.94 121.5) (end 150.94 109.702) (width 0.2) (layer "F.Cu") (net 27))
 (segment (start 158.42 104.339) (end 158.42 97.04) (width 0.2) (layer "F.Cu") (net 27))
 (via (at 158.42 104.339) (size 0.6) (drill 0.3) (layers "F.Cu" "B.Cu") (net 27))
 (via (at 160.768 92.87) (size 0.6) (drill 0.3) (layers "F.Cu" "B.Cu") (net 27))
 (via (at 151.037 109.605) (size 0.6) (drill 0.3) (layers "F.Cu" "B.Cu") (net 27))
 (segment (start 159.572 94.0658) (end 160.768 92.87) (width 0.2) (layer "B.Cu") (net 27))
 (segment (start 153.283 109.605) (end 158.42 104.468) (width 0.2) (layer "B.Cu") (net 27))
 (segment (start 158.42 97.04) (end 158.42 95.8883) (width 0.2) (layer "B.Cu") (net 27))
 (segment (start 158.42 104.468) (end 158.42 104.339) (width 0.2) (layer "B.Cu") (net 27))
 (segment (start 159.572 95.0246) (end 159.572 94.0658) (width 0.2) (layer "B.Cu") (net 27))
 (segment (start 158.708 95.8883) (end 159.572 95.0246) (width 0.2) (layer "B.Cu") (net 27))
 (segment (start 158.42 95.8883) (end 158.708 95.8883) (width 0.2) (layer "B.Cu") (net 27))
 (segment (start 151.037 109.605) (end 153.283 109.605) (width 0.2) (layer "B.Cu") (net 27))
 (segment (start 154.632 70.8034) (end 154.632 85.9137) (width 0.2) (layer "F.Cu") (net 26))
 (segment (start 153.48 68.5) (end 153.48 69.6517) (width 0.2) (layer "F.Cu") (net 26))
 (segment (start 159.718 95.7976) (end 160.96 97.04) (width 0.2) (layer "F.Cu") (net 26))
 (segment (start 154.632 85.9137) (end 159.718 90.9996) (width 0.2) (layer "F.Cu") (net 26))
 (segment (start 159.718 90.9996) (end 159.718 95.7976) (width 0.2) (layer "F.Cu") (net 26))
 (segment (start 153.48 69.6517) (end 154.632 70.8034) (width 0.2) (layer "F.Cu") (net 26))
 (segment (start 149.5 102.5) (end 149.5 108.034) (width 0.2) (layer "F.Cu") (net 31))
 (segment (start 148.798 108.102) (end 148.5 108.4) (width 0.2) (layer "F.Cu") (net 31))
 (segment (start 147.209 102.209) (end 147.209 104.36) (width 0.2) (layer "F.Cu") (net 31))
 (segment (start 147.33 106.634) (end 148.798 108.102) (width 0.2) (layer "F.Cu") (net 31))
 (segment (start 170.5 112.552) (end 169.55 113.502) (width 0.2) (layer "F.Cu") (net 31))
 (segment (start 153.984 112.909) (end 153.984 111.104) (width 0.2) (layer "F.Cu") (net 31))
 (segment (start 155.075 114) (end 153.984 112.909) (width 0.2) (layer "F.Cu") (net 31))
 (segment (start 144.587 99.5876) (end 140.625 103.55) (width 0.2) (layer "F.Cu") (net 31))
 (segment (start 147.33 104.481) (end 147.33 106.634) (width 0.2) (layer "F.Cu") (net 31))
 (segment (start 149.432 108.102) (end 148.798 108.102) (width 0.2) (layer "F.Cu") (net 31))
 (segment (start 147.209 104.36) (end 147.33 104.481) (width 0.2) (layer "F.Cu") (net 31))
 (segment (start 149.432 108.102) (end 149.432 109.125) (width 0.2) (layer "F.Cu") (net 31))
 (segment (start 145.72 97.04) (end 145.72 98.455) (width 0.2) (layer "F.Cu") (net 31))
 (segment (start 144.587 99.5876) (end 147.209 102.209) (width 0.2) (layer "F.Cu") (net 31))
 (segment (start 170.5 112.552) (end 170.5 114) (width 0.2) (layer "F.Cu") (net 31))
 (segment (start 169.55 113.502) (end 169.55 114) (width 0.2) (layer "F.Cu") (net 31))
 (segment (start 170.5 111.104) (end 170.5 112.552) (width 0.2) (layer "F.Cu") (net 31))
 (segment (start 149.5 108.034) (end 149.432 108.102) (width 0.2) (layer "F.Cu") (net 31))
 (segment (start 145.72 98.455) (end 144.587 99.5876) (width 0.2) (layer "F.Cu") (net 31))
 (via (at 153.984 111.104) (size 0.6) (drill 0.3) (layers "F.Cu" "B.Cu") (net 31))
 (via (at 170.5 111.104) (size 0.6) (drill 0.3) (layers "F.Cu" "B.Cu") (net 31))
 (via (at 149.432 109.125) (size 0.6) (drill 0.3) (layers "F.Cu" "B.Cu") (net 31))
 (segment (start 153.984 111.104) (end 151.411 111.104) (width 0.2) (layer "B.Cu") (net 31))
 (segment (start 151.411 111.104) (end 149.432 109.125) (width 0.2) (layer "B.Cu") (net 31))
 (segment (start 170.5 111.104) (end 153.984 111.104) (width 0.2) (layer "B.Cu") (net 31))
 (segment (start 167.4 114) (end 167.315 113.915) (width 0.2) (layer "F.Cu") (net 35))
 (segment (start 166.535 113.915) (end 166.45 114) (width 0.2) (layer "F.Cu") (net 35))
 (segment (start 152 113.5) (end 152.672 113.5) (width 0.2) (layer "F.Cu") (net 35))
 (segment (start 167.315 113.915) (end 166.535 113.915) (width 0.2) (layer "F.Cu") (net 35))
 (segment (start 166.535 113.915) (end 166.411 113.915) (width 0.2) (layer "F.Cu") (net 35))
 (segment (start 152.672 113.5) (end 153.087 113.915) (width 0.2) (layer "F.Cu") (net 35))
 (via (at 153.087 113.915) (size 0.6) (drill 0.3) (layers "F.Cu" "B.Cu") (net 35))
 (via (at 166.411 113.915) (size 0.6) (drill 0.3) (layers "F.Cu" "B.Cu") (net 35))
 (segment (start 166.411 113.915) (end 153.087 113.915) (width 0.2) (layer "B.Cu") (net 35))
 (segment (start 147.811 105.811) (end 147.811 104.111) (width 0.2) (layer "F.Cu") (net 34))
 (segment (start 148.5 106.5) (end 147.811 105.811) (width 0.2) (layer "F.Cu") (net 34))
 (segment (start 153.679 108.309) (end 153.075 107.705) (width 0.2) (layer "F.Cu") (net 34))
 (segment (start 153.075 107.705) (end 153.075 103) (width 0.2) (layer "F.Cu") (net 34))
 (via (at 147.811 104.111) (size 0.6) (drill 0.3) (layers "F.Cu" "B.Cu") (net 34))
 (via (at 153.679 108.309) (size 0.6) (drill 0.3) (layers "F.Cu" "B.Cu") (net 34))
 (segment (start 153.466 108.523) (end 153.679 108.309) (width 0.2) (layer "B.Cu") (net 34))
 (segment (start 143.484 108.016) (end 143.991 108.523) (width 0.2) (layer "B.Cu") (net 34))
 (segment (start 147.811 104.111) (end 146.862 104.111) (width 0.2) (layer "B.Cu") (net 34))
 (segment (start 143.991 108.523) (end 153.466 108.523) (width 0.2) (layer "B.Cu") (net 34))
 (segment (start 146.862 104.111) (end 143.484 107.488) (width 0.2) (layer "B.Cu") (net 34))
 (segment (start 143.484 107.488) (end 143.484 108.016) (width 0.2) (layer "B.Cu") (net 34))
 (segment (start 146.225 106.5) (end 146.609 106.5) (width 0.2) (layer "F.Cu") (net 32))
 (segment (start 146.609 106.5) (end 147.362 107.254) (width 0.2) (layer "F.Cu") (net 32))
 (segment (start 147.362 107.254) (end 147.362 111.788) (width 0.2) (layer "F.Cu") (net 32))
 (segment (start 147.362 111.788) (end 149.075 113.5) (width 0.2) (layer "F.Cu") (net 32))
 (segment (start 142.5 110.273) (end 139 113.773) (width 0.2) (layer "F.Cu") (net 33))
 (segment (start 160.368 114) (end 159.845 114.523) (width 0.2) (layer "F.Cu") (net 33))
 (segment (start 142.5 108.4) (end 146.225 108.4) (width 0.2) (layer "F.Cu") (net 33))
 (segment (start 139 113.773) (end 139 114.5) (width 0.2) (layer "F.Cu") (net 33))
 (segment (start 161.05 114) (end 161.75 114) (width 0.5) (layer "F.Cu") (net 33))
 (segment (start 161.05 114) (end 160.368 114) (width 0.2) (layer "F.Cu") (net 33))
 (segment (start 142.5 104.5) (end 142.5 108.4) (width 0.2) (layer "F.Cu") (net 33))
 (segment (start 142.5 108.4) (end 142.5 110.273) (width 0.2) (layer "F.Cu") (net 33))
 (via (at 159.845 114.523) (size 0.6) (drill 0.3) (layers "F.Cu" "B.Cu") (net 33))
 (segment (start 139.75 114.523) (end 159.845 114.523) (width 0.2) (layer "B.Cu") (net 33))
 (segment (start 139.727 114.5) (end 139.75 114.523) (width 0.2) (layer "B.Cu") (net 33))
 (segment (start 139 114.5) (end 139.727 114.5) (width 0.2) (layer "B.Cu") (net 33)))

